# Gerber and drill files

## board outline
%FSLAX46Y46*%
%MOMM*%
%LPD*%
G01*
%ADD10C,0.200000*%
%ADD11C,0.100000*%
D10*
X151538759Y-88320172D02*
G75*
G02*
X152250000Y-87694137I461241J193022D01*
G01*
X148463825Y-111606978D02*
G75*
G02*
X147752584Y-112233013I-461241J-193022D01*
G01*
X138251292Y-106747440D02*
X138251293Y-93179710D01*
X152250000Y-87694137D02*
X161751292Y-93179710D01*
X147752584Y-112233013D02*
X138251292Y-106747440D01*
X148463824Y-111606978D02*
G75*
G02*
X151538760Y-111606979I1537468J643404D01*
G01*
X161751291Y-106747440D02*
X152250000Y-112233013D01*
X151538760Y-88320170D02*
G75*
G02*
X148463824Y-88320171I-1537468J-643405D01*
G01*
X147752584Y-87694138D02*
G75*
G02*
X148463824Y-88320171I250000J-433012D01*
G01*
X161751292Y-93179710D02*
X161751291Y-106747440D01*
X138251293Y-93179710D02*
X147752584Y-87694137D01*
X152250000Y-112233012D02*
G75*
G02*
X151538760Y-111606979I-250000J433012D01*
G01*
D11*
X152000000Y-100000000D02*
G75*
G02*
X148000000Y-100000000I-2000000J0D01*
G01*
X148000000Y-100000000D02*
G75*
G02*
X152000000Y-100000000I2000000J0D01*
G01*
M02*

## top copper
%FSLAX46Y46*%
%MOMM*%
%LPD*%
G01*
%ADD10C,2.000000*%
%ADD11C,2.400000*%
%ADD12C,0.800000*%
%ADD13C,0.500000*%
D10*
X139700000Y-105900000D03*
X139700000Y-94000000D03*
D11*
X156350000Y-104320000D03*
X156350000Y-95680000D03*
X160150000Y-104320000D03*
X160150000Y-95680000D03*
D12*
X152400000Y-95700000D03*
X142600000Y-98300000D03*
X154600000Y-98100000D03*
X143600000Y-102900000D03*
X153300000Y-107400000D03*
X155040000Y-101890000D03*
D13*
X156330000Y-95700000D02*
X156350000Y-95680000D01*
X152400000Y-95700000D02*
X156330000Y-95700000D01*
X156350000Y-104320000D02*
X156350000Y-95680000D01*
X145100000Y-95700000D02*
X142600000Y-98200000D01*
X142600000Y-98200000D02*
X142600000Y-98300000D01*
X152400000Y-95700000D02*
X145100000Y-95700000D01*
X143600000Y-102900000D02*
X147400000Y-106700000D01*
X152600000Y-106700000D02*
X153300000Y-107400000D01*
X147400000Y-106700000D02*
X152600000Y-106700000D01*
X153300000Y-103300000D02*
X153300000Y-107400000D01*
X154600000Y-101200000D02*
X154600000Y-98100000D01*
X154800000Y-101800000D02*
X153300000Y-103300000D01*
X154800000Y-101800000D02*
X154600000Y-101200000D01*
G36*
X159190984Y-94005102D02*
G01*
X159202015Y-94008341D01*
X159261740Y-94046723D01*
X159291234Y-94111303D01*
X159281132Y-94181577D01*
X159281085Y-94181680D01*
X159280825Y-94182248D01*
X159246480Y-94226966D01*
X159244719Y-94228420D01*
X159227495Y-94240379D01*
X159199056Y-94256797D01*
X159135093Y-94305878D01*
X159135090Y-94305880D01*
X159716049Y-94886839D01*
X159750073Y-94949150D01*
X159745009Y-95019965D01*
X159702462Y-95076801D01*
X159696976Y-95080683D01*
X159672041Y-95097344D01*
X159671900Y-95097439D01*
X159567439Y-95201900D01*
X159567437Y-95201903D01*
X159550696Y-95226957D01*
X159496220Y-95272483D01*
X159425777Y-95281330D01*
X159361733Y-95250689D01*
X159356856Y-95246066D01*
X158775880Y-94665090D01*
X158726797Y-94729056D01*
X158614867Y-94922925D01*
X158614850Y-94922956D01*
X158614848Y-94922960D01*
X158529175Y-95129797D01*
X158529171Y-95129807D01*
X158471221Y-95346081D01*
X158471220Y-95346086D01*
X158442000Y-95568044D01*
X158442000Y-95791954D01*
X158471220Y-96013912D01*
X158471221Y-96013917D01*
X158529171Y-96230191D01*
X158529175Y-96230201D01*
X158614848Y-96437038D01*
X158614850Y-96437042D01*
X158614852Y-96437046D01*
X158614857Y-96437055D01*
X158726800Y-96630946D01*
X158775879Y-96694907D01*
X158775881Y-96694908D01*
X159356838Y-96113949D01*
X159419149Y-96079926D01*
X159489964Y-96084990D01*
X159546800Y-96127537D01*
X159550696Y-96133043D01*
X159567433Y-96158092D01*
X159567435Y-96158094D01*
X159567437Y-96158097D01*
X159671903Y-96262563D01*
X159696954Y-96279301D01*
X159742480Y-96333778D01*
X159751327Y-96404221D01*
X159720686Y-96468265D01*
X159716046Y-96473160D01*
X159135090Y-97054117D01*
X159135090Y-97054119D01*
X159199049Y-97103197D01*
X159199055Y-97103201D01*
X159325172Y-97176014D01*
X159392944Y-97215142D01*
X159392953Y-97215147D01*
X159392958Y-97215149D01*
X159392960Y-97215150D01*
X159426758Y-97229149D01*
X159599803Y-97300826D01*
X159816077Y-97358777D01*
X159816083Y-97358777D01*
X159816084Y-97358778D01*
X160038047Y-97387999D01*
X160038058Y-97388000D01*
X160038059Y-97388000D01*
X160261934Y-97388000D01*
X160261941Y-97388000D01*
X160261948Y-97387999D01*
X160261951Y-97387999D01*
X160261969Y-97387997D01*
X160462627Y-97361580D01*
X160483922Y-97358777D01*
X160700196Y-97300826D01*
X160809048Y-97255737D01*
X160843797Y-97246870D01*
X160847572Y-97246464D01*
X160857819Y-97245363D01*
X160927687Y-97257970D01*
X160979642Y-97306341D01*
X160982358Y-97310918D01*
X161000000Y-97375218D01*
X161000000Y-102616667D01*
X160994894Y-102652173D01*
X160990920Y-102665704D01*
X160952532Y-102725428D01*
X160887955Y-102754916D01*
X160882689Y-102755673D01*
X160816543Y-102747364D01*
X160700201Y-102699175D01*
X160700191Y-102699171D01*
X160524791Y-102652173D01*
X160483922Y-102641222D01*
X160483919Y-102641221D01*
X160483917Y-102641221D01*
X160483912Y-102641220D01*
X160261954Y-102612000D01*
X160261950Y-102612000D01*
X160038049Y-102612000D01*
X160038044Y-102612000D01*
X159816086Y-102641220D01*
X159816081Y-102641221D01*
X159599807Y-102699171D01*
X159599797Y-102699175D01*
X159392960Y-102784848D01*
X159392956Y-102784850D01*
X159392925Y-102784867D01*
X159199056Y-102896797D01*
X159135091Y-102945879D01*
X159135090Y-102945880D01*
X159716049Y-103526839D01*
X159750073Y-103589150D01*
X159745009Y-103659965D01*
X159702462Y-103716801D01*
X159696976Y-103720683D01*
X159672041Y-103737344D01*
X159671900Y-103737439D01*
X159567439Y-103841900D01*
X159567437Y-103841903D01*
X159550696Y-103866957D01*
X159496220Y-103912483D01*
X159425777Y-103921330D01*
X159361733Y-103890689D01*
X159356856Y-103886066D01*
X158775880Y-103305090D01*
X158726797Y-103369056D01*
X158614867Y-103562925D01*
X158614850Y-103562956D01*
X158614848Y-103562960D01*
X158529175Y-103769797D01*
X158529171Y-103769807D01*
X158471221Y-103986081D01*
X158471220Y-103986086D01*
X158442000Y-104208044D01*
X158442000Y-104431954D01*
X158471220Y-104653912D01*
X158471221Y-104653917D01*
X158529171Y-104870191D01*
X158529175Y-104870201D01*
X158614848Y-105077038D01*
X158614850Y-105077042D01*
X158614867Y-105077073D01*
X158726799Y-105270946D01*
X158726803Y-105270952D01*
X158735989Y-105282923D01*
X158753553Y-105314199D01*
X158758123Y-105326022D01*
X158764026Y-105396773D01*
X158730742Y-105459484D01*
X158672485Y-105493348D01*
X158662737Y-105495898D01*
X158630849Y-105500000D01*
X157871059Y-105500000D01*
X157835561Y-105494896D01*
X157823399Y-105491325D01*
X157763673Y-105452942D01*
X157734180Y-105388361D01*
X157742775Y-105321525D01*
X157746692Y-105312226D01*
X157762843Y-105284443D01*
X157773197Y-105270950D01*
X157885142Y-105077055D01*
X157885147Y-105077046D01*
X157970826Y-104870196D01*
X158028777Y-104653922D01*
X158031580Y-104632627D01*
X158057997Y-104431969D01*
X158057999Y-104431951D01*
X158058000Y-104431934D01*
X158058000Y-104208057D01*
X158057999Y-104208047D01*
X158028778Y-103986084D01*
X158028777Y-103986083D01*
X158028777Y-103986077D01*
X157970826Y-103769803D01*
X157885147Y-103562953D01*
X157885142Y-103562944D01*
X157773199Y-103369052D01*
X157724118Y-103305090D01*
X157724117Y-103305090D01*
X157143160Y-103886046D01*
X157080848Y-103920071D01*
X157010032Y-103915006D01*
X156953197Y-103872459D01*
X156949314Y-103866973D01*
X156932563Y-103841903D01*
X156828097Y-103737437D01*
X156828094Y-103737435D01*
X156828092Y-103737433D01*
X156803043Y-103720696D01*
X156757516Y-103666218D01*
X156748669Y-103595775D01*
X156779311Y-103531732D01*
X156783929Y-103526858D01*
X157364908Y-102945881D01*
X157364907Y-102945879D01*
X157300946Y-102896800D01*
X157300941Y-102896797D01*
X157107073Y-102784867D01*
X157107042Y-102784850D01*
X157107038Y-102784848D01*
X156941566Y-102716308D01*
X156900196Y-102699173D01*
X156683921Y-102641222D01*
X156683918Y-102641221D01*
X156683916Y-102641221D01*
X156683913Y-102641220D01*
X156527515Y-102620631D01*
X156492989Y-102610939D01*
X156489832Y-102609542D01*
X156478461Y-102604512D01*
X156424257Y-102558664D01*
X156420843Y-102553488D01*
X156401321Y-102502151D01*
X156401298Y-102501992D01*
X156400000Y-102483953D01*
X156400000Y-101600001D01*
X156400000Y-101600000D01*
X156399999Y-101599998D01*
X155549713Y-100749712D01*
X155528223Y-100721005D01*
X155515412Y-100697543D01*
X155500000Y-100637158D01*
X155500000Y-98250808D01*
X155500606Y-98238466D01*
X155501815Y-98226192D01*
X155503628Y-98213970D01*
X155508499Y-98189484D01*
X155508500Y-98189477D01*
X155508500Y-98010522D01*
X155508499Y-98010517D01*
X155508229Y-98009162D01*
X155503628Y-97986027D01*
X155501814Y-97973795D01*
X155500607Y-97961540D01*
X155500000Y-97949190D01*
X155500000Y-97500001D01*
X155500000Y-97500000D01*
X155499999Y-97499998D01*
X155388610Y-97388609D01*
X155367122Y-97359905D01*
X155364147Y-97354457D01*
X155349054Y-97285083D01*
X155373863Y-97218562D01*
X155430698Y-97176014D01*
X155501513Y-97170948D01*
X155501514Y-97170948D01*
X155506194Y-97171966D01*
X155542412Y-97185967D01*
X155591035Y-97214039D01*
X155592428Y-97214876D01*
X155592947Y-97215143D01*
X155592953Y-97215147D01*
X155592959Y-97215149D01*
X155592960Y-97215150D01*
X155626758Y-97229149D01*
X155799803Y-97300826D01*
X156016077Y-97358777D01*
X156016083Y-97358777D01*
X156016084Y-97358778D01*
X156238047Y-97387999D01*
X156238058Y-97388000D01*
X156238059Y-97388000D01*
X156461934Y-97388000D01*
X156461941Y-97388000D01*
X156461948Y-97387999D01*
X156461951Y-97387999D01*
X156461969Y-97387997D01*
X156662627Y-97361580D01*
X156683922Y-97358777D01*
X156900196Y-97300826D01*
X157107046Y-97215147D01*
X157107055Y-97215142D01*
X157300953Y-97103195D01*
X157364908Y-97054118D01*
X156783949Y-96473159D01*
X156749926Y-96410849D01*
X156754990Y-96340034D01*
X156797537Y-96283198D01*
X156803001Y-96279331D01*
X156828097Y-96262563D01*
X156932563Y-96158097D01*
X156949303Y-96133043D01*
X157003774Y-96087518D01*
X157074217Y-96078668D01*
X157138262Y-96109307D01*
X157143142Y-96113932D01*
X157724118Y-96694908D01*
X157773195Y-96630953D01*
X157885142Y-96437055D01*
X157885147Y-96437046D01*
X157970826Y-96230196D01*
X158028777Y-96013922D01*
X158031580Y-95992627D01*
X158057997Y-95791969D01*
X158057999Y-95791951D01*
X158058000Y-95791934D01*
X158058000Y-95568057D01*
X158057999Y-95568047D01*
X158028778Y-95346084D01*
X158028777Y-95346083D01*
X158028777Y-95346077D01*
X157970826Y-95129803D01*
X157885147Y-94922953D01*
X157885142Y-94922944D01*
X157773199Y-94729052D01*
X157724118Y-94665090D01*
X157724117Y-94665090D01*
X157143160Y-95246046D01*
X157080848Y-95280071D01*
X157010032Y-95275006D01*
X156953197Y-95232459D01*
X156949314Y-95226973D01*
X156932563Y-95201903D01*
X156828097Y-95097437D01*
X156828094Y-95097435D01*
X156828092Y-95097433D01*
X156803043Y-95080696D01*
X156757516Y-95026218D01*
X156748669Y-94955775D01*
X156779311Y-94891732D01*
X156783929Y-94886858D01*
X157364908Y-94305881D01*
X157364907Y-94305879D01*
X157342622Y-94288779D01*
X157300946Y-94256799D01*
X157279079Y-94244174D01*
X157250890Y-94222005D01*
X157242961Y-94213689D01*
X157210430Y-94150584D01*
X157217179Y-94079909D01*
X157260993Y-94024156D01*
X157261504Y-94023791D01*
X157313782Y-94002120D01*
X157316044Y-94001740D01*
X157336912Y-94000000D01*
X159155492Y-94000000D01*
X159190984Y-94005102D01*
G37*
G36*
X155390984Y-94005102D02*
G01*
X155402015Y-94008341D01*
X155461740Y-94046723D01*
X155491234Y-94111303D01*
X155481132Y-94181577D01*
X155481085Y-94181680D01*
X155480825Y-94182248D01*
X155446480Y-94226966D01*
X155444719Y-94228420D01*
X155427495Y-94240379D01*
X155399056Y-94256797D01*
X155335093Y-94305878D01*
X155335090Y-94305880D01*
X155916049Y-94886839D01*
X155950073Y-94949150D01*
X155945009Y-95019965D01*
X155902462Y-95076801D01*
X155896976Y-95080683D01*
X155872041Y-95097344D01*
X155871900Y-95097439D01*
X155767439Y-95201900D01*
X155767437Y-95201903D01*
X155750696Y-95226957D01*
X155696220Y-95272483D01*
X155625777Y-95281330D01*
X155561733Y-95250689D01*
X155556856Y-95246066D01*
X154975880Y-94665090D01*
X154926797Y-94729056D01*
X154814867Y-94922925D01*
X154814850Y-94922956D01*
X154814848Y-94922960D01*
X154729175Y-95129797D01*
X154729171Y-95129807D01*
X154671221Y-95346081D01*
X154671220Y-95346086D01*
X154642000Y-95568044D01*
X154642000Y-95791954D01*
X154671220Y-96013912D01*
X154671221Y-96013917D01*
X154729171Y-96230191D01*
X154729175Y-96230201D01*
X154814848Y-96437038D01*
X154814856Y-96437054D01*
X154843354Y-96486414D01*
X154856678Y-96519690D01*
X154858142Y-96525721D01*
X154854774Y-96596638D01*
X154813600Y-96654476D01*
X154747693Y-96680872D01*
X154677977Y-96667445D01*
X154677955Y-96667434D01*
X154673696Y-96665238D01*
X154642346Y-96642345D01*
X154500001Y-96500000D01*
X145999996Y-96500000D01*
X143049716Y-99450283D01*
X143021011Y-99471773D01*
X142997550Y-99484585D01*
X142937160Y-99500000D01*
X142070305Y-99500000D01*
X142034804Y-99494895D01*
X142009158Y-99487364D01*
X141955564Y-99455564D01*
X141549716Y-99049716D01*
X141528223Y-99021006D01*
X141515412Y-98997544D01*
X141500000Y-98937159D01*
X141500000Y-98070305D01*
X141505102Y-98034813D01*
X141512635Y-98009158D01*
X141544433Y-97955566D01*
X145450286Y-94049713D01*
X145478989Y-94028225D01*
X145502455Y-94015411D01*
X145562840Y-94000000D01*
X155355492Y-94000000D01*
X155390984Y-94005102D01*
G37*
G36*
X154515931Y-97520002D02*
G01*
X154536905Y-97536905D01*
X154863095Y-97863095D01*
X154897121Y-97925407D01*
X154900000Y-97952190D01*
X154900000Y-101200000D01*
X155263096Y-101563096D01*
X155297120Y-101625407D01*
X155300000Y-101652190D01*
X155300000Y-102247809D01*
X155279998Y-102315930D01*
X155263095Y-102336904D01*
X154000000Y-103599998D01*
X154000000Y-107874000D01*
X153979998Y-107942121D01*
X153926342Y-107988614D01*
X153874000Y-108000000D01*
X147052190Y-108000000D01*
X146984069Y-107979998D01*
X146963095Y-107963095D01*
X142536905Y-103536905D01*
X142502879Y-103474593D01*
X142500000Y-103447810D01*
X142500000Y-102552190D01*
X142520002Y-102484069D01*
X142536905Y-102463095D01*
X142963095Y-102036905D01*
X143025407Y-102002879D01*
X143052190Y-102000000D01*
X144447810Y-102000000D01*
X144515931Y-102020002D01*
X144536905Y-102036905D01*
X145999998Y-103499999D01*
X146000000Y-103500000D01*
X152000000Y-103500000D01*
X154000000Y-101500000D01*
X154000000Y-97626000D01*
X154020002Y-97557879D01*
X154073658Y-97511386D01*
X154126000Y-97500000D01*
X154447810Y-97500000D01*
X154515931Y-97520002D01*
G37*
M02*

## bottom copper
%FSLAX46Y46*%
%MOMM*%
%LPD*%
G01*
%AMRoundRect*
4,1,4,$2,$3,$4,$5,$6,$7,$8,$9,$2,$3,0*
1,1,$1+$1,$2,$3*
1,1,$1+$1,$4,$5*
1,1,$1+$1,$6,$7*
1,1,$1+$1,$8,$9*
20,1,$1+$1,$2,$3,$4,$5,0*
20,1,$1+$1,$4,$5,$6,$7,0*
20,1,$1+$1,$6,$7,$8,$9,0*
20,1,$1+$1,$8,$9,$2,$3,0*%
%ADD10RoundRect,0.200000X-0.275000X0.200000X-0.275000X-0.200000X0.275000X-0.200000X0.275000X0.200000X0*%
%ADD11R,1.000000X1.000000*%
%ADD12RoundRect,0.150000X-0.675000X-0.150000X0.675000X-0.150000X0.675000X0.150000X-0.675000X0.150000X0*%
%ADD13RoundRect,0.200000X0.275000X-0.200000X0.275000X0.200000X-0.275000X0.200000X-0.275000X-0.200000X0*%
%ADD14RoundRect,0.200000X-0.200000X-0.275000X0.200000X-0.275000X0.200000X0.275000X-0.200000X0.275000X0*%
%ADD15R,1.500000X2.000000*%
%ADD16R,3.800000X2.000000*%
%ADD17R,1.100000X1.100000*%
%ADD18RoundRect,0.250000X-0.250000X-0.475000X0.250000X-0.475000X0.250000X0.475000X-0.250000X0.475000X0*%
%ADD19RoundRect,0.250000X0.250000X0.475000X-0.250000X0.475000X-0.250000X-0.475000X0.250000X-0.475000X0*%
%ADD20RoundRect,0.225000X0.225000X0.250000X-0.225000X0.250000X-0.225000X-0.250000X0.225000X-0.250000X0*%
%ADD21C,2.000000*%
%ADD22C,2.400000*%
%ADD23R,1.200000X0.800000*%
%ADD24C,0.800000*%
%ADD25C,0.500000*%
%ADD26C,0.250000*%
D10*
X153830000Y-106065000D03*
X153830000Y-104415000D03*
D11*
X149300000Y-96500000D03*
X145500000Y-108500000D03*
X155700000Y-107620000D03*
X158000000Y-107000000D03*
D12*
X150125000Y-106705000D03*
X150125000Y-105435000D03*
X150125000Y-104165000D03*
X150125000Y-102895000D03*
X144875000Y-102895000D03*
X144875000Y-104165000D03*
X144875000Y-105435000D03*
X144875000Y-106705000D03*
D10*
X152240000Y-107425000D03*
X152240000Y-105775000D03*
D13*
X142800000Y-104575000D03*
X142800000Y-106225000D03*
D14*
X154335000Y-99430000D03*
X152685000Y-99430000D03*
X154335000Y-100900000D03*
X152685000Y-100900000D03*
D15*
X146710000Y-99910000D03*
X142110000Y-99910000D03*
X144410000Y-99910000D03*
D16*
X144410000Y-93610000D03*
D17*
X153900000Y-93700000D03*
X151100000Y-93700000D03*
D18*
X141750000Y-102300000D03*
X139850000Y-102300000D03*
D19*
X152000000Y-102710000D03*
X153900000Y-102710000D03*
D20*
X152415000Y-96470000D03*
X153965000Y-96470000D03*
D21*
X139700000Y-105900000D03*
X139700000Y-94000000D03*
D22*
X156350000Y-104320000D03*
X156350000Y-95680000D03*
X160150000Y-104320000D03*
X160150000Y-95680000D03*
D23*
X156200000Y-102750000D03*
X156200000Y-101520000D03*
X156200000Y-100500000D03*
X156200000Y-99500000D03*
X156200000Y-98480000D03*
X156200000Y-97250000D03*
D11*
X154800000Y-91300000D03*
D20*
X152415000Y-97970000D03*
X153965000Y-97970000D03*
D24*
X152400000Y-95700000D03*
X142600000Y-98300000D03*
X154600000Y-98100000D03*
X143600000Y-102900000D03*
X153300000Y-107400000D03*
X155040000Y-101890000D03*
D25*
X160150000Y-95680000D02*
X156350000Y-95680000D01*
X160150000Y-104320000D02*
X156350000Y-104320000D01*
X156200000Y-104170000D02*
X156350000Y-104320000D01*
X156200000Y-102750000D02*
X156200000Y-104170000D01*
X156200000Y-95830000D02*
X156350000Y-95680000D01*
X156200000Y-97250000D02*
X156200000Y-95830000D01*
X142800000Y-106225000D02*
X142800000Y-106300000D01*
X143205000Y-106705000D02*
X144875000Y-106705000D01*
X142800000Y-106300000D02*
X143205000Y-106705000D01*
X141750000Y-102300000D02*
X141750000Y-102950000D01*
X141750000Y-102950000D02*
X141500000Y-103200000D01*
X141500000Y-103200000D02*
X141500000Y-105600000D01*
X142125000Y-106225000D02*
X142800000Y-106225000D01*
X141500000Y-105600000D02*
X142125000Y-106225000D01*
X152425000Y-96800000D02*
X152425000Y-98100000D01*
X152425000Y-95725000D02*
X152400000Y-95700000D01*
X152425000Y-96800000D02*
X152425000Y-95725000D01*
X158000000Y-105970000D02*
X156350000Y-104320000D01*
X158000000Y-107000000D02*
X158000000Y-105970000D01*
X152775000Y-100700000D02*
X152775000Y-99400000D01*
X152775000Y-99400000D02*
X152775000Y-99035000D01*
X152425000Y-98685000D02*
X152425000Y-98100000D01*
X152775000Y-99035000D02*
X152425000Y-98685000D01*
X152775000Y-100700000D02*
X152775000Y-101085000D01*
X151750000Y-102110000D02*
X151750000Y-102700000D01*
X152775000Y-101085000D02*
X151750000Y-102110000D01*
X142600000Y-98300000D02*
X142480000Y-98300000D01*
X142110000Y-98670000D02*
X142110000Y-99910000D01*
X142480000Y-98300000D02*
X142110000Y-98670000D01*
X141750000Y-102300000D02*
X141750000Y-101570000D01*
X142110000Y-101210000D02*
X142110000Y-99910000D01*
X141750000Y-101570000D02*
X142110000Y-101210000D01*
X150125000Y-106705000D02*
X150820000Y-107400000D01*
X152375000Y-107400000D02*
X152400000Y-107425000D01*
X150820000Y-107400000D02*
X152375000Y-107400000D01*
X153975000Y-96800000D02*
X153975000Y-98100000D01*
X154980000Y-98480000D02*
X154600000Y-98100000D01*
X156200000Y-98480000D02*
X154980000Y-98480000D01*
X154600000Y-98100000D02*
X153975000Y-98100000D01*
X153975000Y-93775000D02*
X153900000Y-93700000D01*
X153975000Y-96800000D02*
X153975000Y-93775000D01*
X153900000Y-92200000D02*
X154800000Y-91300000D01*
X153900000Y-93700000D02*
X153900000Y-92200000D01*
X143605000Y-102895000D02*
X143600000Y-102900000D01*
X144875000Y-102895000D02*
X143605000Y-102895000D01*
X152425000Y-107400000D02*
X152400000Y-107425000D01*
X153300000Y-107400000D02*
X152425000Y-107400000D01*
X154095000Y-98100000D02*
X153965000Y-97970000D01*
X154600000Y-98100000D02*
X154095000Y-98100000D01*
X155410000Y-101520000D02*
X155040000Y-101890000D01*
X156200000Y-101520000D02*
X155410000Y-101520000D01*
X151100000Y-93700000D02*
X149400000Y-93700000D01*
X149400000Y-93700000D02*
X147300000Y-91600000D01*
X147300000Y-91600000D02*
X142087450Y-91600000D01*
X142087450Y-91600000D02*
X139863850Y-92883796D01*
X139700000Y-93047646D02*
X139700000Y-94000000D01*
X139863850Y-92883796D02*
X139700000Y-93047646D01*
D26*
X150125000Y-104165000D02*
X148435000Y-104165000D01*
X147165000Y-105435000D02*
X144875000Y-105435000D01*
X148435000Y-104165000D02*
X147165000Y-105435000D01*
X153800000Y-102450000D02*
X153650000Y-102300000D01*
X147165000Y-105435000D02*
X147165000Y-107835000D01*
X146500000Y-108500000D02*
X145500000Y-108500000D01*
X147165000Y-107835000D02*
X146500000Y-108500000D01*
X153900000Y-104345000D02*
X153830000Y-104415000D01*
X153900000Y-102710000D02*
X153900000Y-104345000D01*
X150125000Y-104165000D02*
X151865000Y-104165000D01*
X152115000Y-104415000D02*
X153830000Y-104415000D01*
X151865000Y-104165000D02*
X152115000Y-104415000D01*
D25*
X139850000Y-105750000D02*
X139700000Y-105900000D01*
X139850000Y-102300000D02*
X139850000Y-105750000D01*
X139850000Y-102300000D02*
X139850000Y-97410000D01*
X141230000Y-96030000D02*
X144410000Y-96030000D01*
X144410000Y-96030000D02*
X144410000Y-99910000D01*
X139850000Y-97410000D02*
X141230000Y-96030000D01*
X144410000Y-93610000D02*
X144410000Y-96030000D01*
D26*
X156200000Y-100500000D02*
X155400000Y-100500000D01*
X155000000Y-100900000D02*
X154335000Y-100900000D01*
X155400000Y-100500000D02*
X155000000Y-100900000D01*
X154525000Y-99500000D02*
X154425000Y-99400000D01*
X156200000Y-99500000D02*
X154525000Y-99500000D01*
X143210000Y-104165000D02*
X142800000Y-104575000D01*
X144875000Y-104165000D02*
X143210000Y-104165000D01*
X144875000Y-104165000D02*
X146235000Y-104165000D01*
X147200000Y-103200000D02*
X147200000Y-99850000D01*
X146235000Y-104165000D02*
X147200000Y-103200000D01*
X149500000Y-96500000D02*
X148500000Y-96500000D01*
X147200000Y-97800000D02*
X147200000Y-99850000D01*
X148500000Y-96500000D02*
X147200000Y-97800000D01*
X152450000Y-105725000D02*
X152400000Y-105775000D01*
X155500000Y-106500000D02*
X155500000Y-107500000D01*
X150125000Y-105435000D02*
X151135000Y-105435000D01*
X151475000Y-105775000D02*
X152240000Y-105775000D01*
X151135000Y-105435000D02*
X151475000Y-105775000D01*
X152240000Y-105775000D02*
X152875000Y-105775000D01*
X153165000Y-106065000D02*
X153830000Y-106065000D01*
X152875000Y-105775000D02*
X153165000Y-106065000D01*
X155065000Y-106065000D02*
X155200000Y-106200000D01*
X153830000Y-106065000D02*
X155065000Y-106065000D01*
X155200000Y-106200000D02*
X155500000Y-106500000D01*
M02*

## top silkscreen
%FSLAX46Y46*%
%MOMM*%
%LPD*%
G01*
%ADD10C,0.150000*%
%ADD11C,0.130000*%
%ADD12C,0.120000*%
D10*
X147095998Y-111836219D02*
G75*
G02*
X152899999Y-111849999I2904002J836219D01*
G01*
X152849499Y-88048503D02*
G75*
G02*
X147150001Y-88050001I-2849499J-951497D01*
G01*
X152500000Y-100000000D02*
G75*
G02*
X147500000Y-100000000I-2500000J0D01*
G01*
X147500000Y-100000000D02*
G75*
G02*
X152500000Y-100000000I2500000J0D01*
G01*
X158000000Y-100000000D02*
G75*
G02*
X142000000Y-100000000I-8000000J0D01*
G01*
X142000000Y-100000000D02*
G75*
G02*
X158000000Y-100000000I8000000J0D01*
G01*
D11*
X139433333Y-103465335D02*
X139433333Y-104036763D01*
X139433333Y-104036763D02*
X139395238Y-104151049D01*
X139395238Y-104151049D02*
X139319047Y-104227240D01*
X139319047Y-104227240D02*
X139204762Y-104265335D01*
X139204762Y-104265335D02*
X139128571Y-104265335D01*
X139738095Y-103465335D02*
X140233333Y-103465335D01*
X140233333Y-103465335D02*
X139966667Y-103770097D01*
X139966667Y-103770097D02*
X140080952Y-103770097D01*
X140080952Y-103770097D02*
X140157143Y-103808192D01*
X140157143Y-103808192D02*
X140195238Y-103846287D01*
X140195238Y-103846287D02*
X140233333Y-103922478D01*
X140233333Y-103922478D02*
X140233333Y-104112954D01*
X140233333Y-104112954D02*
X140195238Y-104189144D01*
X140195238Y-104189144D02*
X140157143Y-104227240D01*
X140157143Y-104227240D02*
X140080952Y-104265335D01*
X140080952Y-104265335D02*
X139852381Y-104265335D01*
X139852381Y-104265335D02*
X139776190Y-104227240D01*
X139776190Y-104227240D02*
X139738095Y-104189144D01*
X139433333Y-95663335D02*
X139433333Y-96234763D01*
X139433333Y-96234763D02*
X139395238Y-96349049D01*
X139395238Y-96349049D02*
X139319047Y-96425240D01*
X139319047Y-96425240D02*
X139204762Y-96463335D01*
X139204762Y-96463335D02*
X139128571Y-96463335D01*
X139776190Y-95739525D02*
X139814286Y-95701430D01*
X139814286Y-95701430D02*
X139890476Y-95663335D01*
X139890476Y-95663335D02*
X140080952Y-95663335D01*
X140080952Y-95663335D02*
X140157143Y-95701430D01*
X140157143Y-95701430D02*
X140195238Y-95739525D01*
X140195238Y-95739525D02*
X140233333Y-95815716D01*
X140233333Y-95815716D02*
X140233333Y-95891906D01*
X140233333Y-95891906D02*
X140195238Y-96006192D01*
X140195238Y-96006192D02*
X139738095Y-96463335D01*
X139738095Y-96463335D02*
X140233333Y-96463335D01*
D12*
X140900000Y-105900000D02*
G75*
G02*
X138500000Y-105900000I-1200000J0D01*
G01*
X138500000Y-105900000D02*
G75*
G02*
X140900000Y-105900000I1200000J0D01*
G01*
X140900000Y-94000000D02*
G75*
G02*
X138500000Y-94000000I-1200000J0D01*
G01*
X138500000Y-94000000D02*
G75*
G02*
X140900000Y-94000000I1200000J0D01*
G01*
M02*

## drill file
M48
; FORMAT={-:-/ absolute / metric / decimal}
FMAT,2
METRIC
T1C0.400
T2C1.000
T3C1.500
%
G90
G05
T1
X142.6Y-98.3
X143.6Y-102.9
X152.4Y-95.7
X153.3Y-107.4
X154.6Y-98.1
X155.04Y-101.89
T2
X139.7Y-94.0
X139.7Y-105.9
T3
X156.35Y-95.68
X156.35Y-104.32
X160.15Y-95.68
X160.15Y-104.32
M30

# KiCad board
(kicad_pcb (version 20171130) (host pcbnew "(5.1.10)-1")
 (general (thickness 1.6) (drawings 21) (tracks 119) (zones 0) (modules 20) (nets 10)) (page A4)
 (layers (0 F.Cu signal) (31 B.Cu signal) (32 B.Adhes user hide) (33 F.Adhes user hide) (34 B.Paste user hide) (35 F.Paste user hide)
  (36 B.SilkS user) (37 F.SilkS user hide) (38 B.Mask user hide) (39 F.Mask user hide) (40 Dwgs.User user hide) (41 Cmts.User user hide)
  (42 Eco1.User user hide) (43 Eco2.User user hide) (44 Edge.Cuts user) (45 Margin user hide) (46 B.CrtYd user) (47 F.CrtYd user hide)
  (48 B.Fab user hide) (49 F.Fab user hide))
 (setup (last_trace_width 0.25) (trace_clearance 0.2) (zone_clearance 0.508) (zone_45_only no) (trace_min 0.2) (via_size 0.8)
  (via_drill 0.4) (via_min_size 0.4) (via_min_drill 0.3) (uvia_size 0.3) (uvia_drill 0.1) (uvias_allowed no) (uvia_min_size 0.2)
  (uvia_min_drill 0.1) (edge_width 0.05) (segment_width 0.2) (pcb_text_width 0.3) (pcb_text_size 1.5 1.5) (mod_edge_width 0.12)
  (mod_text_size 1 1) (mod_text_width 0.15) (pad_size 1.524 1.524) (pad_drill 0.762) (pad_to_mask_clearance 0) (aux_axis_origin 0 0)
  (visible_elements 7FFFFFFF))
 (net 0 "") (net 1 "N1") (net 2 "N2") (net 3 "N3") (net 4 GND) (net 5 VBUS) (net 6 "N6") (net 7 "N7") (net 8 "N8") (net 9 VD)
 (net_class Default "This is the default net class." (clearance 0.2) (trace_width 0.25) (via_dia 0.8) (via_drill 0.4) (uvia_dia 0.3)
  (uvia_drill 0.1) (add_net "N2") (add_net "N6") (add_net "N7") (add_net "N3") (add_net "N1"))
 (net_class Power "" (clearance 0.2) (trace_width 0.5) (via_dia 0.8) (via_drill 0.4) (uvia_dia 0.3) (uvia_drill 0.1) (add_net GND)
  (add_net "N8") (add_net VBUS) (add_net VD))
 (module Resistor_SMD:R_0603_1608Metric (layer B.Cu) (at 153.83 105.24 270)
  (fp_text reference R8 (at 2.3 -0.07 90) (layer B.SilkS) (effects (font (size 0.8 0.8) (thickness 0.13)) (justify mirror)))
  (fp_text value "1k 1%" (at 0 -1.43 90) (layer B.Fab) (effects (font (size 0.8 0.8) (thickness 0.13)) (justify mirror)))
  (pad 2 smd roundrect (at 0.825 0 270) (size 0.8 0.95) (layers B.Cu B.Paste B.Mask) (roundrect_rratio 0.25) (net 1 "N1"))
  (pad 1 smd roundrect (at -0.825 0 270) (size 0.8 0.95) (layers B.Cu B.Paste B.Mask) (roundrect_rratio 0.25) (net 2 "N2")))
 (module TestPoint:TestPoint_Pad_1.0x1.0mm (layer B.Cu) (at 149.3 96.5)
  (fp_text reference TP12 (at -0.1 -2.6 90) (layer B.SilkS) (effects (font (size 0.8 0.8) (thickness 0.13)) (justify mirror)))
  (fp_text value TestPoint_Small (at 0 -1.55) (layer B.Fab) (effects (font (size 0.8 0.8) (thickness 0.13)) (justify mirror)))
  (pad 1 smd rect (at 0 0) (size 1 1) (layers B.Cu B.Mask) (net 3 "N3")))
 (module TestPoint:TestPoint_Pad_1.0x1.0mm (layer B.Cu) (at 145.5 108.5)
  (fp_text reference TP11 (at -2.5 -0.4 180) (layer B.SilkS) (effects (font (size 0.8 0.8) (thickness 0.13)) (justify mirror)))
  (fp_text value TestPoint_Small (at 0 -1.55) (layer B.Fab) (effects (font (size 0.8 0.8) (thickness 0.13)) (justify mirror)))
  (pad 1 smd rect (at 0 0) (size 1 1) (layers B.Cu B.Mask) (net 2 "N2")))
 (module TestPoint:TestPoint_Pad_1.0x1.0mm (layer B.Cu) (at 155.7 107.62)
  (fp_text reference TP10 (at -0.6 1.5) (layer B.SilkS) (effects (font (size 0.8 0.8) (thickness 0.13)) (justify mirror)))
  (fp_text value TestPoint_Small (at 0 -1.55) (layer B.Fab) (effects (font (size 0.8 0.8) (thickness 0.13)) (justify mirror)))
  (pad 1 smd rect (at 0 0) (size 1 1) (layers B.Cu B.Mask) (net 1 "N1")))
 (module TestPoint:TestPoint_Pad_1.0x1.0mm (layer B.Cu) (at 158 107)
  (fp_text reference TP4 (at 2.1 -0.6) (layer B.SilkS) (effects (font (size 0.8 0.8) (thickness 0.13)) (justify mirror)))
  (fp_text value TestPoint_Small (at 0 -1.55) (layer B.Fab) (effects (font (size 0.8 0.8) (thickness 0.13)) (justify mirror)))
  (pad 1 smd rect (at 0 0) (size 1 1) (layers B.Cu B.Mask) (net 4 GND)))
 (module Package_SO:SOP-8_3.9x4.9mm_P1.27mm (layer B.Cu) (at 147.5 104.8)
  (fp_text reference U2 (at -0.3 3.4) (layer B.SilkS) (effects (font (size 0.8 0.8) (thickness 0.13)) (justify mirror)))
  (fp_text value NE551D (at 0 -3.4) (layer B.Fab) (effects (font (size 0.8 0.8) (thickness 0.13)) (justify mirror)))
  (pad 8 smd roundrect (at 2.625 1.905) (size 1.65 0.6) (layers B.Cu B.Paste B.Mask) (roundrect_rratio 0.25) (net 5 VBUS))
  (pad 7 smd roundrect (at 2.625 0.635) (size 1.65 0.6) (layers B.Cu B.Paste B.Mask) (roundrect_rratio 0.25) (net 1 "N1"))
  (pad 6 smd roundrect (at 2.625 -0.635) (size 1.65 0.6) (layers B.Cu B.Paste B.Mask) (roundrect_rratio 0.25) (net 2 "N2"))
  (pad 5 smd roundrect (at 2.625 -1.905) (size 1.65 0.6) (layers B.Cu B.Paste B.Mask) (roundrect_rratio 0.25))
  (pad 4 smd roundrect (at -2.625 -1.905) (size 1.65 0.6) (layers B.Cu B.Paste B.Mask) (roundrect_rratio 0.25) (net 5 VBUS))
  (pad 3 smd roundrect (at -2.625 -0.635) (size 1.65 0.6) (layers B.Cu B.Paste B.Mask) (roundrect_rratio 0.25) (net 3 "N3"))
  (pad 2 smd roundrect (at -2.625 0.635) (size 1.65 0.6) (layers B.Cu B.Paste B.Mask) (roundrect_rratio 0.25) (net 2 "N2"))
  (pad 1 smd roundrect (at -2.625 1.905) (size 1.65 0.6) (layers B.Cu B.Paste B.Mask) (roundrect_rratio 0.25) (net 4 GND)))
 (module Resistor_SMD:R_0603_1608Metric (layer B.Cu) (at 152.24 106.6 270)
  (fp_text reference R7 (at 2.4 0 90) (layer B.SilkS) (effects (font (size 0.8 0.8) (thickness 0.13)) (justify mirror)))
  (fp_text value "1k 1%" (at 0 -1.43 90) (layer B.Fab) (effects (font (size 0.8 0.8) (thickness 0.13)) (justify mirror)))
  (pad 2 smd roundrect (at 0.825 0 270) (size 0.8 0.95) (layers B.Cu B.Paste B.Mask) (roundrect_rratio 0.25) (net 5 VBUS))
  (pad 1 smd roundrect (at -0.825 0 270) (size 0.8 0.95) (layers B.Cu B.Paste B.Mask) (roundrect_rratio 0.25) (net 1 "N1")))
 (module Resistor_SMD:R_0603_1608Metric (layer B.Cu) (at 142.8 105.4 90)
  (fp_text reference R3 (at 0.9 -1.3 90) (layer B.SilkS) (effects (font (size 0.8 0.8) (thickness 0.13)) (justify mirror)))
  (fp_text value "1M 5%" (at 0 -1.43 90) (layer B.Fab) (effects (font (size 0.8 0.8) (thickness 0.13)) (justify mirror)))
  (pad 2 smd roundrect (at 0.825 0 90) (size 0.8 0.95) (layers B.Cu B.Paste B.Mask) (roundrect_rratio 0.25) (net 3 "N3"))
  (pad 1 smd roundrect (at -0.825 0 90) (size 0.8 0.95) (layers B.Cu B.Paste B.Mask) (roundrect_rratio 0.25) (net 4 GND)))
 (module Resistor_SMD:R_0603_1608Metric (layer B.Cu) (at 153.51 99.43)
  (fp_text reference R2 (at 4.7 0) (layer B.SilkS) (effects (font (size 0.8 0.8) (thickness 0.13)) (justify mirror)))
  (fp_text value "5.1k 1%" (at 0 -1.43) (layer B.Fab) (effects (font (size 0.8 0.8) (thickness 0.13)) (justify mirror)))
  (pad 2 smd roundrect (at 0.825 0) (size 0.8 0.95) (layers B.Cu B.Paste B.Mask) (roundrect_rratio 0.25) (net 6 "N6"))
  (pad 1 smd roundrect (at -0.825 0) (size 0.8 0.95) (layers B.Cu B.Paste B.Mask) (roundrect_rratio 0.25) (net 4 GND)))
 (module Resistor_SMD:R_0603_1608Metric (layer B.Cu) (at 153.51 100.9)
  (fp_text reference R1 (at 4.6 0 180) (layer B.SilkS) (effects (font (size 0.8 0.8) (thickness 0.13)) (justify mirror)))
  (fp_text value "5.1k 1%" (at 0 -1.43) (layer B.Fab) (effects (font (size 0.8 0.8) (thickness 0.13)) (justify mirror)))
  (pad 2 smd roundrect (at 0.825 0) (size 0.8 0.95) (layers B.Cu B.Paste B.Mask) (roundrect_rratio 0.25) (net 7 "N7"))
  (pad 1 smd roundrect (at -0.825 0) (size 0.8 0.95) (layers B.Cu B.Paste B.Mask) (roundrect_rratio 0.25) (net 4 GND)))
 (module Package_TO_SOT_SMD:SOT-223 (layer B.Cu) (at 144.41 96.76 90)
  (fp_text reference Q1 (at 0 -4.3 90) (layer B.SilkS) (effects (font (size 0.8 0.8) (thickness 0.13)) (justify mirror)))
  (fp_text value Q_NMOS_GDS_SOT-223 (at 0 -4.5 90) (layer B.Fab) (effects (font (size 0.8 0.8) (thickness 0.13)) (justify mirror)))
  (pad 1 smd rect (at -3.15 2.3 90) (size 2 1.5) (layers B.Cu B.Paste B.Mask) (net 3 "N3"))
  (pad 3 smd rect (at -3.15 -2.3 90) (size 2 1.5) (layers B.Cu B.Paste B.Mask) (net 4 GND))
  (pad 2 smd rect (at -3.15 0 90) (size 2 1.5) (layers B.Cu B.Paste B.Mask) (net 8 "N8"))
  (pad 4 smd rect (at 3.15 0 90) (size 2 3.8) (layers B.Cu B.Paste B.Mask) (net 8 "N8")))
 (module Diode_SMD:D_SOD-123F (layer B.Cu) (at 152.5 93.7)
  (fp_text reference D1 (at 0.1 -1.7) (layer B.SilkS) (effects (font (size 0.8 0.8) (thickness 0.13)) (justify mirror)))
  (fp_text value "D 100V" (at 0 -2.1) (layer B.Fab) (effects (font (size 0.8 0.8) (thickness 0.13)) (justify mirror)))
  (pad 2 smd rect (at 1.4 0) (size 1.1 1.1) (layers B.Cu B.Paste B.Mask) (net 5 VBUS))
  (pad 1 smd rect (at -1.4 0) (size 1.1 1.1) (layers B.Cu B.Paste B.Mask) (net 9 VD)))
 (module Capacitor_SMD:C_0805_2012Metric (layer B.Cu) (at 140.8 102.3)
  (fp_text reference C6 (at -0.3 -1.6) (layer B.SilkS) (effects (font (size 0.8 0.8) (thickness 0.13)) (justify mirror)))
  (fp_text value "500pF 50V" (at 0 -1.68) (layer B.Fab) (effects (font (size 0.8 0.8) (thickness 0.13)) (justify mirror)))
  (pad 2 smd roundrect (at 0.95 0) (size 1 1.45) (layers B.Cu B.Paste B.Mask) (roundrect_rratio 0.25) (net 4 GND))
  (pad 1 smd roundrect (at -0.95 0) (size 1 1.45) (layers B.Cu B.Paste B.Mask) (roundrect_rratio 0.25) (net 8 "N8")))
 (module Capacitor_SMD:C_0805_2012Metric (layer B.Cu) (at 152.95 102.71 180)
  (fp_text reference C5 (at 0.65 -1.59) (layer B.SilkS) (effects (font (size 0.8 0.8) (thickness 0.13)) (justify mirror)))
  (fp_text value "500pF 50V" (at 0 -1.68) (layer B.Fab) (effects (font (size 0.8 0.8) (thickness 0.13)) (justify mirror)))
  (pad 2 smd roundrect (at 0.95 0 180) (size 1 1.45) (layers B.Cu B.Paste B.Mask) (roundrect_rratio 0.25) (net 4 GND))
  (pad 1 smd roundrect (at -0.95 0 180) (size 1 1.45) (layers B.Cu B.Paste B.Mask) (roundrect_rratio 0.25) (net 2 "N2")))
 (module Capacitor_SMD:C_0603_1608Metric (layer B.Cu) (at 153.19 96.47 180)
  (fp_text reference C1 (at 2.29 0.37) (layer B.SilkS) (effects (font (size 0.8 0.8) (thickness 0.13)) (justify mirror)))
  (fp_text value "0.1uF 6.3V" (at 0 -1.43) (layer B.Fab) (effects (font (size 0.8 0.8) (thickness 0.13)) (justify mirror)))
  (pad 2 smd roundrect (at 0.775 0 180) (size 0.9 0.95) (layers B.Cu B.Paste B.Mask) (roundrect_rratio 0.25) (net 4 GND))
  (pad 1 smd roundrect (at -0.775 0 180) (size 0.9 0.95) (layers B.Cu B.Paste B.Mask) (roundrect_rratio 0.25) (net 5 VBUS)))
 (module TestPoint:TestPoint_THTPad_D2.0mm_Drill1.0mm (layer F.Cu) (at 139.7 105.9)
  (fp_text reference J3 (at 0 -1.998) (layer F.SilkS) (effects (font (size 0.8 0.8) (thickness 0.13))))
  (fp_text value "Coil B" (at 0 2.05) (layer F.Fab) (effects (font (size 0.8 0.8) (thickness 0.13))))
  (fp_circle (center 0 0) (end 0 1.2) (layer F.SilkS) (width 0.12))
  (pad 1 thru_hole circle (at 0 0) (size 2 2) (drill 1) (layers *.Cu *.Mask) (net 8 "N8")))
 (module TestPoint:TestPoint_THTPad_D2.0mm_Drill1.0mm (layer F.Cu) (at 139.7 94)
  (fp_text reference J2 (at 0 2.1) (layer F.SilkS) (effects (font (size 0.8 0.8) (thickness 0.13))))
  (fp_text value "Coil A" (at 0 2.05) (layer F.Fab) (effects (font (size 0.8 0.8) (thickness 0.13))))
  (fp_circle (center 0 0) (end 0 1.2) (layer F.SilkS) (width 0.12))
  (pad 1 thru_hole circle (at 0 0) (size 2 2) (drill 1) (layers *.Cu *.Mask) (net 9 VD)))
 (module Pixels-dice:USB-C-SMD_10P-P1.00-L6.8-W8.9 (layer B.Cu) (at 158.35 100)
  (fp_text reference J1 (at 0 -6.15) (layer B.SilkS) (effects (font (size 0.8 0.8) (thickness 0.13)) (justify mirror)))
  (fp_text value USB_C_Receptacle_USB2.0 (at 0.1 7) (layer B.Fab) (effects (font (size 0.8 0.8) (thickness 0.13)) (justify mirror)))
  (pad S1 thru_hole circle (at -2 4.32 270) (size 2.4 2.4) (drill 1.5) (layers *.Cu *.Mask) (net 4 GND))
  (pad S1 thru_hole circle (at -2 -4.32 270) (size 2.4 2.4) (drill 1.5) (layers *.Cu *.Mask) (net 4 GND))
  (pad S1 thru_hole circle (at 1.8 4.32 270) (size 2.4 2.4) (drill 1.5) (layers *.Cu *.Mask) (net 4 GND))
  (pad S1 thru_hole circle (at 1.8 -4.32 270) (size 2.4 2.4) (drill 1.5) (layers *.Cu *.Mask) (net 4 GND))
  (pad A12 smd rect (at -2.15 2.75 270) (size 0.8 1.2) (layers B.Cu B.Paste B.Mask) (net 4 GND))
  (pad A9 smd rect (at -2.15 1.52 270) (size 0.8 1.2) (layers B.Cu B.Paste B.Mask) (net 5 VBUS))
  (pad B5 smd rect (at -2.15 0.5 270) (size 0.8 1.2) (layers B.Cu B.Paste B.Mask) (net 7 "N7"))
  (pad A5 smd rect (at -2.15 -0.5 270) (size 0.8 1.2) (layers B.Cu B.Paste B.Mask) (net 6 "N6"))
  (pad B9 smd rect (at -2.15 -1.52 270) (size 0.8 1.2) (layers B.Cu B.Paste B.Mask) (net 5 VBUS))
  (pad B12 smd rect (at -2.15 -2.75 270) (size 0.8 1.2) (layers B.Cu B.Paste B.Mask) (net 4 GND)))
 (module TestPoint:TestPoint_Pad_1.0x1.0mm (layer B.Cu) (at 154.8 91.3)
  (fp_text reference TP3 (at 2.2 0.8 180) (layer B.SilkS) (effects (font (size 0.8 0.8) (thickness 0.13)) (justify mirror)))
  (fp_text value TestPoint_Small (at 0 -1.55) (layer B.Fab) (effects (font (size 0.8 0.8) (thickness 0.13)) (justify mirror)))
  (pad 1 smd rect (at 0 0) (size 1 1) (layers B.Cu B.Mask) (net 5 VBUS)))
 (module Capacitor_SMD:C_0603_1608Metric (layer B.Cu) (at 153.19 97.97 180)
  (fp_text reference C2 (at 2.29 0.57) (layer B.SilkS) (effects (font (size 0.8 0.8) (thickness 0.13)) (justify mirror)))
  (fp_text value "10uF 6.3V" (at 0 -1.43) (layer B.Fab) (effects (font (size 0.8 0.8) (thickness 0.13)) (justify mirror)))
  (pad 2 smd roundrect (at 0.775 0 180) (size 0.9 0.95) (layers B.Cu B.Paste B.Mask) (roundrect_rratio 0.25) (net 4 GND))
  (pad 1 smd roundrect (at -0.775 0 180) (size 0.9 0.95) (layers B.Cu B.Paste B.Mask) (roundrect_rratio 0.25) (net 5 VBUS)))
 (gr_arc (start 150 111) (end 152.899999 111.849999) (angle -212.4) (layer F.SilkS) (width 0.15))
 (gr_arc (start 150 89) (end 147.150001 88.050001) (angle -216.9) (layer F.SilkS) (width 0.15))
 (gr_arc (start 152 88.12715) (end 152.25 87.694137) (angle -142.7084941) (layer Edge.Cuts) (width 0.2))
 (gr_arc (start 148.002584 111.8) (end 147.752584 112.233013) (angle -142.7084941) (layer Edge.Cuts) (width 0.2))
 (gr_line (start 138.251292 106.74744) (end 138.251293 93.17971) (layer Edge.Cuts) (width 0.2))
 (gr_line (start 152.25 87.694137) (end 161.751292 93.17971) (layer Edge.Cuts) (width 0.2))
 (gr_line (start 147.752584 112.233013) (end 138.251292 106.74744) (layer Edge.Cuts) (width 0.2))
 (gr_arc (start 150.001292 110.963574) (end 151.53876 111.606979) (angle -225.4169678) (layer Edge.Cuts) (width 0.2))
 (gr_line (start 161.751291 106.74744) (end 152.25 112.233013) (layer Edge.Cuts) (width 0.2))
 (gr_arc (start 150.001292 88.963575) (end 148.463824 88.320171) (angle -225.4169678) (layer Edge.Cuts) (width 0.2))
 (gr_arc (start 148.002584 88.12715) (end 148.463824 88.320171) (angle -142.7084738) (layer Edge.Cuts) (width 0.2))
 (gr_line (start 161.751292 93.17971) (end 161.751291 106.74744) (layer Edge.Cuts) (width 0.2))
 (gr_line (start 138.251293 93.17971) (end 147.752584 87.694137) (layer Edge.Cuts) (width 0.2))
 (gr_arc (start 152 111.8) (end 151.53876 111.606979) (angle -142.7084738) (layer Edge.Cuts) (width 0.2))
 (gr_circle (center 150 100) (end 152 100) (layer Edge.Cuts) (width 0.1))
 (gr_circle (center 150 100) (end 152.5 100) (layer F.SilkS) (width 0.15))
 (gr_circle (center 150 100) (end 158 100) (layer F.SilkS) (width 0.15))
 (segment (start 160.15 95.68) (end 156.35 95.68) (width 0.5) (layer B.Cu) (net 4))
 (segment (start 160.15 104.32) (end 156.35 104.32) (width 0.5) (layer B.Cu) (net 4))
 (segment (start 156.2 104.17) (end 156.35 104.32) (width 0.5) (layer B.Cu) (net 4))
 (segment (start 156.2 102.75) (end 156.2 104.17) (width 0.5) (layer B.Cu) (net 4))
 (segment (start 156.2 95.83) (end 156.35 95.68) (width 0.5) (layer B.Cu) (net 4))
 (segment (start 156.2 97.25) (end 156.2 95.83) (width 0.5) (layer B.Cu) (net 4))
 (segment (start 142.8 106.225) (end 142.8 106.3) (width 0.5) (layer B.Cu) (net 4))
 (segment (start 143.205 106.705) (end 144.875 106.705) (width 0.5) (layer B.Cu) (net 4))
 (segment (start 142.8 106.3) (end 143.205 106.705) (width 0.5) (layer B.Cu) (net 4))
 (segment (start 141.75 102.3) (end 141.75 102.95) (width 0.5) (layer B.Cu) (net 4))
 (segment (start 141.75 102.95) (end 141.5 103.2) (width 0.5) (layer B.Cu) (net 4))
 (segment (start 141.5 103.2) (end 141.5 105.6) (width 0.5) (layer B.Cu) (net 4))
 (segment (start 142.125 106.225) (end 142.8 106.225) (width 0.5) (layer B.Cu) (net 4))
 (segment (start 141.5 105.6) (end 142.125 106.225) (width 0.5) (layer B.Cu) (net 4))
 (segment (start 152.425 96.8) (end 152.425 98.1) (width 0.5) (layer B.Cu) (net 4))
 (via (at 152.4 95.7) (size 0.8) (drill 0.4) (layers F.Cu B.Cu) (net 4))
 (segment (start 152.425 95.725) (end 152.4 95.7) (width 0.5) (layer B.Cu) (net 4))
 (segment (start 152.425 96.8) (end 152.425 95.725) (width 0.5) (layer B.Cu) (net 4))
 (segment (start 156.33 95.7) (end 156.35 95.68) (width 0.5) (layer F.Cu) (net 4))
 (segment (start 152.4 95.7) (end 156.33 95.7) (width 0.5) (layer F.Cu) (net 4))
 (segment (start 156.35 104.32) (end 156.35 95.68) (width 0.5) (layer F.Cu) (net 4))
 (segment (start 158 105.97) (end 156.35 104.32) (width 0.5) (layer B.Cu) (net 4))
 (segment (start 158 107) (end 158 105.97) (width 0.5) (layer B.Cu) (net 4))
 (via (at 142.6 98.3) (size 0.8) (drill 0.4) (layers F.Cu B.Cu) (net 4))
 (segment (start 145.1 95.7) (end 142.6 98.2) (width 0.5) (layer F.Cu) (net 4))
 (segment (start 142.6 98.2) (end 142.6 98.3) (width 0.5) (layer F.Cu) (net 4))
 (segment (start 152.4 95.7) (end 145.1 95.7) (width 0.5) (layer F.Cu) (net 4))
 (segment (start 152.775 100.7) (end 152.775 99.4) (width 0.5) (layer B.Cu) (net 4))
 (segment (start 152.775 99.4) (end 152.775 99.035) (width 0.5) (layer B.Cu) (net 4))
 (segment (start 152.425 98.685) (end 152.425 98.1) (width 0.5) (layer B.Cu) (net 4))
 (segment (start 152.775 99.035) (end 152.425 98.685) (width 0.5) (layer B.Cu) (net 4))
 (segment (start 152.775 100.7) (end 152.775 101.085) (width 0.5) (layer B.Cu) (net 4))
 (segment (start 151.75 102.11) (end 151.75 102.7) (width 0.5) (layer B.Cu) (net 4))
 (segment (start 152.775 101.085) (end 151.75 102.11) (width 0.5) (layer B.Cu) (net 4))
 (segment (start 142.6 98.3) (end 142.48 98.3) (width 0.5) (layer B.Cu) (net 4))
 (segment (start 142.11 98.67) (end 142.11 99.91) (width 0.5) (layer B.Cu) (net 4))
 (segment (start 142.48 98.3) (end 142.11 98.67) (width 0.5) (layer B.Cu) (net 4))
 (segment (start 141.75 102.3) (end 141.75 101.57) (width 0.5) (layer B.Cu) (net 4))
 (segment (start 142.11 101.21) (end 142.11 99.91) (width 0.5) (layer B.Cu) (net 4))
 (segment (start 141.75 101.57) (end 142.11 101.21) (width 0.5) (layer B.Cu) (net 4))
 (segment (start 150.125 106.705) (end 150.82 107.4) (width 0.5) (layer B.Cu) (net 5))
 (segment (start 152.375 107.4) (end 152.4 107.425) (width 0.5) (layer B.Cu) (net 5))
 (segment (start 150.82 107.4) (end 152.375 107.4) (width 0.5) (layer B.Cu) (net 5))
 (segment (start 153.975 96.8) (end 153.975 98.1) (width 0.5) (layer B.Cu) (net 5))
 (via (at 154.6 98.1) (size 0.8) (drill 0.4) (layers F.Cu B.Cu) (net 5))
 (segment (start 154.98 98.48) (end 154.6 98.1) (width 0.5) (layer B.Cu) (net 5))
 (segment (start 156.2 98.48) (end 154.98 98.48) (width 0.5) (layer B.Cu) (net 5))
 (segment (start 154.6 98.1) (end 153.975 98.1) (width 0.5) (layer B.Cu) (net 5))
 (segment (start 153.975 93.775) (end 153.9 93.7) (width 0.5) (layer B.Cu) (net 5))
 (segment (start 153.975 96.8) (end 153.975 93.775) (width 0.5) (layer B.Cu) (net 5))
 (segment (start 153.9 92.2) (end 154.8 91.3) (width 0.5) (layer B.Cu) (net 5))
 (segment (start 153.9 93.7) (end 153.9 92.2) (width 0.5) (layer B.Cu) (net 5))
 (via (at 143.6 102.9) (size 0.8) (drill 0.4) (layers F.Cu B.Cu) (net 5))
 (segment (start 143.605 102.895) (end 143.6 102.9) (width 0.5) (layer B.Cu) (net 5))
 (segment (start 144.875 102.895) (end 143.605 102.895) (width 0.5) (layer B.Cu) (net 5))
 (segment (start 143.6 102.9) (end 147.4 106.7) (width 0.5) (layer F.Cu) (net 5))
 (via (at 153.3 107.4) (size 0.8) (drill 0.4) (layers F.Cu B.Cu) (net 5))
 (segment (start 152.6 106.7) (end 153.3 107.4) (width 0.5) (layer F.Cu) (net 5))
 (segment (start 147.4 106.7) (end 152.6 106.7) (width 0.5) (layer F.Cu) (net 5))
 (segment (start 152.425 107.4) (end 152.4 107.425) (width 0.5) (layer B.Cu) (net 5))
 (segment (start 153.3 107.4) (end 152.425 107.4) (width 0.5) (layer B.Cu) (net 5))
 (segment (start 153.3 103.3) (end 153.3 107.4) (width 0.5) (layer F.Cu) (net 5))
 (segment (start 154.6 101.2) (end 154.6 98.1) (width 0.5) (layer F.Cu) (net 5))
 (segment (start 154.8 101.8) (end 153.3 103.3) (width 0.5) (layer F.Cu) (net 5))
 (segment (start 154.8 101.8) (end 154.6 101.2) (width 0.5) (layer F.Cu) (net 5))
 (via (at 155.04 101.89) (size 0.8) (drill 0.4) (layers F.Cu B.Cu) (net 5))
 (segment (start 154.095 98.1) (end 153.965 97.97) (width 0.5) (layer B.Cu) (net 5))
 (segment (start 154.6 98.1) (end 154.095 98.1) (width 0.5) (layer B.Cu) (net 5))
 (segment (start 155.41 101.52) (end 155.04 101.89) (width 0.5) (layer B.Cu) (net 5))
 (segment (start 156.2 101.52) (end 155.41 101.52) (width 0.5) (layer B.Cu) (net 5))
 (segment (start 151.1 93.7) (end 149.4 93.7) (width 0.5) (layer B.Cu) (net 9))
 (segment (start 149.4 93.7) (end 147.3 91.6) (width 0.5) (layer B.Cu) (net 9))
 (segment (start 147.3 91.6) (end 142.08745 91.6) (width 0.5) (layer B.Cu) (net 9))
 (segment (start 142.08745 91.6) (end 139.86385 92.883796) (width 0.5) (layer B.Cu) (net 9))
 (segment (start 139.7 93.047646) (end 139.7 94) (width 0.5) (layer B.Cu) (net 9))
 (segment (start 139.86385 92.883796) (end 139.7 93.047646) (width 0.5) (layer B.Cu) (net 9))
 (segment (start 150.125 104.165) (end 148.435 104.165) (width 0.25) (layer B.Cu) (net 2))
 (segment (start 147.165 105.435) (end 144.875 105.435) (width 0.25) (layer B.Cu) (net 2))
 (segment (start 148.435 104.165) (end 147.165 105.435) (width 0.25) (layer B.Cu) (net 2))
 (segment (start 153.8 102.45) (end 153.65 102.3) (width 0.25) (layer B.Cu) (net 2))
 (segment (start 147.165 105.435) (end 147.165 107.835) (width 0.25) (layer B.Cu) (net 2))
 (segment (start 146.5 108.5) (end 145.5 108.5) (width 0.25) (layer B.Cu) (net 2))
 (segment (start 147.165 107.835) (end 146.5 108.5) (width 0.25) (layer B.Cu) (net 2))
 (segment (start 153.9 104.345) (end 153.83 104.415) (width 0.25) (layer B.Cu) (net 2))
 (segment (start 153.9 102.71) (end 153.9 104.345) (width 0.25) (layer B.Cu) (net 2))
 (segment (start 150.125 104.165) (end 151.865 104.165) (width 0.25) (layer B.Cu) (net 2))
 (segment (start 152.115 104.415) (end 153.83 104.415) (width 0.25) (layer B.Cu) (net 2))
 (segment (start 151.865 104.165) (end 152.115 104.415) (width 0.25) (layer B.Cu) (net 2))
 (segment (start 139.85 105.75) (end 139.7 105.9) (width 0.5) (layer B.Cu) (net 8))
 (segment (start 139.85 102.3) (end 139.85 105.75) (width 0.5) (layer B.Cu) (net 8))
 (segment (start 139.85 102.3) (end 139.85 97.41) (width 0.5) (layer B.Cu) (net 8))
 (segment (start 141.23 96.03) (end 144.41 96.03) (width 0.5) (layer B.Cu) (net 8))
 (segment (start 144.41 96.03) (end 144.41 99.91) (width 0.5) (layer B.Cu) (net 8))
 (segment (start 139.85 97.41) (end 141.23 96.03) (width 0.5) (layer B.Cu) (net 8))
 (segment (start 144.41 93.61) (end 144.41 96.03) (width 0.5) (layer B.Cu) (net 8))
 (segment (start 156.2 100.5) (end 155.4 100.5) (width 0.25) (layer B.Cu) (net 7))
 (segment (start 155 100.9) (end 154.335 100.9) (width 0.25) (layer B.Cu) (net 7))
 (segment (start 155.4 100.5) (end 155 100.9) (width 0.25) (layer B.Cu) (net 7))
 (segment (start 154.525 99.5) (end 154.425 99.4) (width 0.25) (layer B.Cu) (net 6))
 (segment (start 156.2 99.5) (end 154.525 99.5) (width 0.25) (layer B.Cu) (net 6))
 (segment (start 143.21 104.165) (end 142.8 104.575) (width 0.25) (layer B.Cu) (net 3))
 (segment (start 144.875 104.165) (end 143.21 104.165) (width 0.25) (layer B.Cu) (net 3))
 (segment (start 144.875 104.165) (end 146.235 104.165) (width 0.25) (layer B.Cu) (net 3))
 (segment (start 147.2 103.2) (end 147.2 99.85) (width 0.25) (layer B.Cu) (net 3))
 (segment (start 146.235 104.165) (end 147.2 103.2) (width 0.25) (layer B.Cu) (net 3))
 (segment (start 149.5 96.5) (end 148.5 96.5) (width 0.25) (layer B.Cu) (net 3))
 (segment (start 147.2 97.8) (end 147.2 99.85) (width 0.25) (layer B.Cu) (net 3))
 (segment (start 148.5 96.5) (end 147.2 97.8) (width 0.25) (layer B.Cu) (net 3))
 (segment (start 152.45 105.725) (end 152.4 105.775) (width 0.25) (layer B.Cu) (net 1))
 (segment (start 155.5 106.5) (end 155.5 107.5) (width 0.25) (layer B.Cu) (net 1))
 (segment (start 150.125 105.435) (end 151.135 105.435) (width 0.25) (layer B.Cu) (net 1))
 (segment (start 151.475 105.775) (end 152.24 105.775) (width 0.25) (layer B.Cu) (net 1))
 (segment (start 151.135 105.435) (end 151.475 105.775) (width 0.25) (layer B.Cu) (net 1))
 (segment (start 152.24 105.775) (end 152.875 105.775) (width 0.25) (layer B.Cu) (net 1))
 (segment (start 153.165 106.065) (end 153.83 106.065) (width 0.25) (layer B.Cu) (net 1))
 (segment (start 152.875 105.775) (end 153.165 106.065) (width 0.25) (layer B.Cu) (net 1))
 (segment (start 155.065 106.065) (end 155.2 106.2) (width 0.25) (layer B.Cu) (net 1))
 (segment (start 153.83 106.065) (end 155.065 106.065) (width 0.25) (layer B.Cu) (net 1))
 (segment (start 155.2 106.2) (end 155.5 106.5) (width 0.25) (layer B.Cu) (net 1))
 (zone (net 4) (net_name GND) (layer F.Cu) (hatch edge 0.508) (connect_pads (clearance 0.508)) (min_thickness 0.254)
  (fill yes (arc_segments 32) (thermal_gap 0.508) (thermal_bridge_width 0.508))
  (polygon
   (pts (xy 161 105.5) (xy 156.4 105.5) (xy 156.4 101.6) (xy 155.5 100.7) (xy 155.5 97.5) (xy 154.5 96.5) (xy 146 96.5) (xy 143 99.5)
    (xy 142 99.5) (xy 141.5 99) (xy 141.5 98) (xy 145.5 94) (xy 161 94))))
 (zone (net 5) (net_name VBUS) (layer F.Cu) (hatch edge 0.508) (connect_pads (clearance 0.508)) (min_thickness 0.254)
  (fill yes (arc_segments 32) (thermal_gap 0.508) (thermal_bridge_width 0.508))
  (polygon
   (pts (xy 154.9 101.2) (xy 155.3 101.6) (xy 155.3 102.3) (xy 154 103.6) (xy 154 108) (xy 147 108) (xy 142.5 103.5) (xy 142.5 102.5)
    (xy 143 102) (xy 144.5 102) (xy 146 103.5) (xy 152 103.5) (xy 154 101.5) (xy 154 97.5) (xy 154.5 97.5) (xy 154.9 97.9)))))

